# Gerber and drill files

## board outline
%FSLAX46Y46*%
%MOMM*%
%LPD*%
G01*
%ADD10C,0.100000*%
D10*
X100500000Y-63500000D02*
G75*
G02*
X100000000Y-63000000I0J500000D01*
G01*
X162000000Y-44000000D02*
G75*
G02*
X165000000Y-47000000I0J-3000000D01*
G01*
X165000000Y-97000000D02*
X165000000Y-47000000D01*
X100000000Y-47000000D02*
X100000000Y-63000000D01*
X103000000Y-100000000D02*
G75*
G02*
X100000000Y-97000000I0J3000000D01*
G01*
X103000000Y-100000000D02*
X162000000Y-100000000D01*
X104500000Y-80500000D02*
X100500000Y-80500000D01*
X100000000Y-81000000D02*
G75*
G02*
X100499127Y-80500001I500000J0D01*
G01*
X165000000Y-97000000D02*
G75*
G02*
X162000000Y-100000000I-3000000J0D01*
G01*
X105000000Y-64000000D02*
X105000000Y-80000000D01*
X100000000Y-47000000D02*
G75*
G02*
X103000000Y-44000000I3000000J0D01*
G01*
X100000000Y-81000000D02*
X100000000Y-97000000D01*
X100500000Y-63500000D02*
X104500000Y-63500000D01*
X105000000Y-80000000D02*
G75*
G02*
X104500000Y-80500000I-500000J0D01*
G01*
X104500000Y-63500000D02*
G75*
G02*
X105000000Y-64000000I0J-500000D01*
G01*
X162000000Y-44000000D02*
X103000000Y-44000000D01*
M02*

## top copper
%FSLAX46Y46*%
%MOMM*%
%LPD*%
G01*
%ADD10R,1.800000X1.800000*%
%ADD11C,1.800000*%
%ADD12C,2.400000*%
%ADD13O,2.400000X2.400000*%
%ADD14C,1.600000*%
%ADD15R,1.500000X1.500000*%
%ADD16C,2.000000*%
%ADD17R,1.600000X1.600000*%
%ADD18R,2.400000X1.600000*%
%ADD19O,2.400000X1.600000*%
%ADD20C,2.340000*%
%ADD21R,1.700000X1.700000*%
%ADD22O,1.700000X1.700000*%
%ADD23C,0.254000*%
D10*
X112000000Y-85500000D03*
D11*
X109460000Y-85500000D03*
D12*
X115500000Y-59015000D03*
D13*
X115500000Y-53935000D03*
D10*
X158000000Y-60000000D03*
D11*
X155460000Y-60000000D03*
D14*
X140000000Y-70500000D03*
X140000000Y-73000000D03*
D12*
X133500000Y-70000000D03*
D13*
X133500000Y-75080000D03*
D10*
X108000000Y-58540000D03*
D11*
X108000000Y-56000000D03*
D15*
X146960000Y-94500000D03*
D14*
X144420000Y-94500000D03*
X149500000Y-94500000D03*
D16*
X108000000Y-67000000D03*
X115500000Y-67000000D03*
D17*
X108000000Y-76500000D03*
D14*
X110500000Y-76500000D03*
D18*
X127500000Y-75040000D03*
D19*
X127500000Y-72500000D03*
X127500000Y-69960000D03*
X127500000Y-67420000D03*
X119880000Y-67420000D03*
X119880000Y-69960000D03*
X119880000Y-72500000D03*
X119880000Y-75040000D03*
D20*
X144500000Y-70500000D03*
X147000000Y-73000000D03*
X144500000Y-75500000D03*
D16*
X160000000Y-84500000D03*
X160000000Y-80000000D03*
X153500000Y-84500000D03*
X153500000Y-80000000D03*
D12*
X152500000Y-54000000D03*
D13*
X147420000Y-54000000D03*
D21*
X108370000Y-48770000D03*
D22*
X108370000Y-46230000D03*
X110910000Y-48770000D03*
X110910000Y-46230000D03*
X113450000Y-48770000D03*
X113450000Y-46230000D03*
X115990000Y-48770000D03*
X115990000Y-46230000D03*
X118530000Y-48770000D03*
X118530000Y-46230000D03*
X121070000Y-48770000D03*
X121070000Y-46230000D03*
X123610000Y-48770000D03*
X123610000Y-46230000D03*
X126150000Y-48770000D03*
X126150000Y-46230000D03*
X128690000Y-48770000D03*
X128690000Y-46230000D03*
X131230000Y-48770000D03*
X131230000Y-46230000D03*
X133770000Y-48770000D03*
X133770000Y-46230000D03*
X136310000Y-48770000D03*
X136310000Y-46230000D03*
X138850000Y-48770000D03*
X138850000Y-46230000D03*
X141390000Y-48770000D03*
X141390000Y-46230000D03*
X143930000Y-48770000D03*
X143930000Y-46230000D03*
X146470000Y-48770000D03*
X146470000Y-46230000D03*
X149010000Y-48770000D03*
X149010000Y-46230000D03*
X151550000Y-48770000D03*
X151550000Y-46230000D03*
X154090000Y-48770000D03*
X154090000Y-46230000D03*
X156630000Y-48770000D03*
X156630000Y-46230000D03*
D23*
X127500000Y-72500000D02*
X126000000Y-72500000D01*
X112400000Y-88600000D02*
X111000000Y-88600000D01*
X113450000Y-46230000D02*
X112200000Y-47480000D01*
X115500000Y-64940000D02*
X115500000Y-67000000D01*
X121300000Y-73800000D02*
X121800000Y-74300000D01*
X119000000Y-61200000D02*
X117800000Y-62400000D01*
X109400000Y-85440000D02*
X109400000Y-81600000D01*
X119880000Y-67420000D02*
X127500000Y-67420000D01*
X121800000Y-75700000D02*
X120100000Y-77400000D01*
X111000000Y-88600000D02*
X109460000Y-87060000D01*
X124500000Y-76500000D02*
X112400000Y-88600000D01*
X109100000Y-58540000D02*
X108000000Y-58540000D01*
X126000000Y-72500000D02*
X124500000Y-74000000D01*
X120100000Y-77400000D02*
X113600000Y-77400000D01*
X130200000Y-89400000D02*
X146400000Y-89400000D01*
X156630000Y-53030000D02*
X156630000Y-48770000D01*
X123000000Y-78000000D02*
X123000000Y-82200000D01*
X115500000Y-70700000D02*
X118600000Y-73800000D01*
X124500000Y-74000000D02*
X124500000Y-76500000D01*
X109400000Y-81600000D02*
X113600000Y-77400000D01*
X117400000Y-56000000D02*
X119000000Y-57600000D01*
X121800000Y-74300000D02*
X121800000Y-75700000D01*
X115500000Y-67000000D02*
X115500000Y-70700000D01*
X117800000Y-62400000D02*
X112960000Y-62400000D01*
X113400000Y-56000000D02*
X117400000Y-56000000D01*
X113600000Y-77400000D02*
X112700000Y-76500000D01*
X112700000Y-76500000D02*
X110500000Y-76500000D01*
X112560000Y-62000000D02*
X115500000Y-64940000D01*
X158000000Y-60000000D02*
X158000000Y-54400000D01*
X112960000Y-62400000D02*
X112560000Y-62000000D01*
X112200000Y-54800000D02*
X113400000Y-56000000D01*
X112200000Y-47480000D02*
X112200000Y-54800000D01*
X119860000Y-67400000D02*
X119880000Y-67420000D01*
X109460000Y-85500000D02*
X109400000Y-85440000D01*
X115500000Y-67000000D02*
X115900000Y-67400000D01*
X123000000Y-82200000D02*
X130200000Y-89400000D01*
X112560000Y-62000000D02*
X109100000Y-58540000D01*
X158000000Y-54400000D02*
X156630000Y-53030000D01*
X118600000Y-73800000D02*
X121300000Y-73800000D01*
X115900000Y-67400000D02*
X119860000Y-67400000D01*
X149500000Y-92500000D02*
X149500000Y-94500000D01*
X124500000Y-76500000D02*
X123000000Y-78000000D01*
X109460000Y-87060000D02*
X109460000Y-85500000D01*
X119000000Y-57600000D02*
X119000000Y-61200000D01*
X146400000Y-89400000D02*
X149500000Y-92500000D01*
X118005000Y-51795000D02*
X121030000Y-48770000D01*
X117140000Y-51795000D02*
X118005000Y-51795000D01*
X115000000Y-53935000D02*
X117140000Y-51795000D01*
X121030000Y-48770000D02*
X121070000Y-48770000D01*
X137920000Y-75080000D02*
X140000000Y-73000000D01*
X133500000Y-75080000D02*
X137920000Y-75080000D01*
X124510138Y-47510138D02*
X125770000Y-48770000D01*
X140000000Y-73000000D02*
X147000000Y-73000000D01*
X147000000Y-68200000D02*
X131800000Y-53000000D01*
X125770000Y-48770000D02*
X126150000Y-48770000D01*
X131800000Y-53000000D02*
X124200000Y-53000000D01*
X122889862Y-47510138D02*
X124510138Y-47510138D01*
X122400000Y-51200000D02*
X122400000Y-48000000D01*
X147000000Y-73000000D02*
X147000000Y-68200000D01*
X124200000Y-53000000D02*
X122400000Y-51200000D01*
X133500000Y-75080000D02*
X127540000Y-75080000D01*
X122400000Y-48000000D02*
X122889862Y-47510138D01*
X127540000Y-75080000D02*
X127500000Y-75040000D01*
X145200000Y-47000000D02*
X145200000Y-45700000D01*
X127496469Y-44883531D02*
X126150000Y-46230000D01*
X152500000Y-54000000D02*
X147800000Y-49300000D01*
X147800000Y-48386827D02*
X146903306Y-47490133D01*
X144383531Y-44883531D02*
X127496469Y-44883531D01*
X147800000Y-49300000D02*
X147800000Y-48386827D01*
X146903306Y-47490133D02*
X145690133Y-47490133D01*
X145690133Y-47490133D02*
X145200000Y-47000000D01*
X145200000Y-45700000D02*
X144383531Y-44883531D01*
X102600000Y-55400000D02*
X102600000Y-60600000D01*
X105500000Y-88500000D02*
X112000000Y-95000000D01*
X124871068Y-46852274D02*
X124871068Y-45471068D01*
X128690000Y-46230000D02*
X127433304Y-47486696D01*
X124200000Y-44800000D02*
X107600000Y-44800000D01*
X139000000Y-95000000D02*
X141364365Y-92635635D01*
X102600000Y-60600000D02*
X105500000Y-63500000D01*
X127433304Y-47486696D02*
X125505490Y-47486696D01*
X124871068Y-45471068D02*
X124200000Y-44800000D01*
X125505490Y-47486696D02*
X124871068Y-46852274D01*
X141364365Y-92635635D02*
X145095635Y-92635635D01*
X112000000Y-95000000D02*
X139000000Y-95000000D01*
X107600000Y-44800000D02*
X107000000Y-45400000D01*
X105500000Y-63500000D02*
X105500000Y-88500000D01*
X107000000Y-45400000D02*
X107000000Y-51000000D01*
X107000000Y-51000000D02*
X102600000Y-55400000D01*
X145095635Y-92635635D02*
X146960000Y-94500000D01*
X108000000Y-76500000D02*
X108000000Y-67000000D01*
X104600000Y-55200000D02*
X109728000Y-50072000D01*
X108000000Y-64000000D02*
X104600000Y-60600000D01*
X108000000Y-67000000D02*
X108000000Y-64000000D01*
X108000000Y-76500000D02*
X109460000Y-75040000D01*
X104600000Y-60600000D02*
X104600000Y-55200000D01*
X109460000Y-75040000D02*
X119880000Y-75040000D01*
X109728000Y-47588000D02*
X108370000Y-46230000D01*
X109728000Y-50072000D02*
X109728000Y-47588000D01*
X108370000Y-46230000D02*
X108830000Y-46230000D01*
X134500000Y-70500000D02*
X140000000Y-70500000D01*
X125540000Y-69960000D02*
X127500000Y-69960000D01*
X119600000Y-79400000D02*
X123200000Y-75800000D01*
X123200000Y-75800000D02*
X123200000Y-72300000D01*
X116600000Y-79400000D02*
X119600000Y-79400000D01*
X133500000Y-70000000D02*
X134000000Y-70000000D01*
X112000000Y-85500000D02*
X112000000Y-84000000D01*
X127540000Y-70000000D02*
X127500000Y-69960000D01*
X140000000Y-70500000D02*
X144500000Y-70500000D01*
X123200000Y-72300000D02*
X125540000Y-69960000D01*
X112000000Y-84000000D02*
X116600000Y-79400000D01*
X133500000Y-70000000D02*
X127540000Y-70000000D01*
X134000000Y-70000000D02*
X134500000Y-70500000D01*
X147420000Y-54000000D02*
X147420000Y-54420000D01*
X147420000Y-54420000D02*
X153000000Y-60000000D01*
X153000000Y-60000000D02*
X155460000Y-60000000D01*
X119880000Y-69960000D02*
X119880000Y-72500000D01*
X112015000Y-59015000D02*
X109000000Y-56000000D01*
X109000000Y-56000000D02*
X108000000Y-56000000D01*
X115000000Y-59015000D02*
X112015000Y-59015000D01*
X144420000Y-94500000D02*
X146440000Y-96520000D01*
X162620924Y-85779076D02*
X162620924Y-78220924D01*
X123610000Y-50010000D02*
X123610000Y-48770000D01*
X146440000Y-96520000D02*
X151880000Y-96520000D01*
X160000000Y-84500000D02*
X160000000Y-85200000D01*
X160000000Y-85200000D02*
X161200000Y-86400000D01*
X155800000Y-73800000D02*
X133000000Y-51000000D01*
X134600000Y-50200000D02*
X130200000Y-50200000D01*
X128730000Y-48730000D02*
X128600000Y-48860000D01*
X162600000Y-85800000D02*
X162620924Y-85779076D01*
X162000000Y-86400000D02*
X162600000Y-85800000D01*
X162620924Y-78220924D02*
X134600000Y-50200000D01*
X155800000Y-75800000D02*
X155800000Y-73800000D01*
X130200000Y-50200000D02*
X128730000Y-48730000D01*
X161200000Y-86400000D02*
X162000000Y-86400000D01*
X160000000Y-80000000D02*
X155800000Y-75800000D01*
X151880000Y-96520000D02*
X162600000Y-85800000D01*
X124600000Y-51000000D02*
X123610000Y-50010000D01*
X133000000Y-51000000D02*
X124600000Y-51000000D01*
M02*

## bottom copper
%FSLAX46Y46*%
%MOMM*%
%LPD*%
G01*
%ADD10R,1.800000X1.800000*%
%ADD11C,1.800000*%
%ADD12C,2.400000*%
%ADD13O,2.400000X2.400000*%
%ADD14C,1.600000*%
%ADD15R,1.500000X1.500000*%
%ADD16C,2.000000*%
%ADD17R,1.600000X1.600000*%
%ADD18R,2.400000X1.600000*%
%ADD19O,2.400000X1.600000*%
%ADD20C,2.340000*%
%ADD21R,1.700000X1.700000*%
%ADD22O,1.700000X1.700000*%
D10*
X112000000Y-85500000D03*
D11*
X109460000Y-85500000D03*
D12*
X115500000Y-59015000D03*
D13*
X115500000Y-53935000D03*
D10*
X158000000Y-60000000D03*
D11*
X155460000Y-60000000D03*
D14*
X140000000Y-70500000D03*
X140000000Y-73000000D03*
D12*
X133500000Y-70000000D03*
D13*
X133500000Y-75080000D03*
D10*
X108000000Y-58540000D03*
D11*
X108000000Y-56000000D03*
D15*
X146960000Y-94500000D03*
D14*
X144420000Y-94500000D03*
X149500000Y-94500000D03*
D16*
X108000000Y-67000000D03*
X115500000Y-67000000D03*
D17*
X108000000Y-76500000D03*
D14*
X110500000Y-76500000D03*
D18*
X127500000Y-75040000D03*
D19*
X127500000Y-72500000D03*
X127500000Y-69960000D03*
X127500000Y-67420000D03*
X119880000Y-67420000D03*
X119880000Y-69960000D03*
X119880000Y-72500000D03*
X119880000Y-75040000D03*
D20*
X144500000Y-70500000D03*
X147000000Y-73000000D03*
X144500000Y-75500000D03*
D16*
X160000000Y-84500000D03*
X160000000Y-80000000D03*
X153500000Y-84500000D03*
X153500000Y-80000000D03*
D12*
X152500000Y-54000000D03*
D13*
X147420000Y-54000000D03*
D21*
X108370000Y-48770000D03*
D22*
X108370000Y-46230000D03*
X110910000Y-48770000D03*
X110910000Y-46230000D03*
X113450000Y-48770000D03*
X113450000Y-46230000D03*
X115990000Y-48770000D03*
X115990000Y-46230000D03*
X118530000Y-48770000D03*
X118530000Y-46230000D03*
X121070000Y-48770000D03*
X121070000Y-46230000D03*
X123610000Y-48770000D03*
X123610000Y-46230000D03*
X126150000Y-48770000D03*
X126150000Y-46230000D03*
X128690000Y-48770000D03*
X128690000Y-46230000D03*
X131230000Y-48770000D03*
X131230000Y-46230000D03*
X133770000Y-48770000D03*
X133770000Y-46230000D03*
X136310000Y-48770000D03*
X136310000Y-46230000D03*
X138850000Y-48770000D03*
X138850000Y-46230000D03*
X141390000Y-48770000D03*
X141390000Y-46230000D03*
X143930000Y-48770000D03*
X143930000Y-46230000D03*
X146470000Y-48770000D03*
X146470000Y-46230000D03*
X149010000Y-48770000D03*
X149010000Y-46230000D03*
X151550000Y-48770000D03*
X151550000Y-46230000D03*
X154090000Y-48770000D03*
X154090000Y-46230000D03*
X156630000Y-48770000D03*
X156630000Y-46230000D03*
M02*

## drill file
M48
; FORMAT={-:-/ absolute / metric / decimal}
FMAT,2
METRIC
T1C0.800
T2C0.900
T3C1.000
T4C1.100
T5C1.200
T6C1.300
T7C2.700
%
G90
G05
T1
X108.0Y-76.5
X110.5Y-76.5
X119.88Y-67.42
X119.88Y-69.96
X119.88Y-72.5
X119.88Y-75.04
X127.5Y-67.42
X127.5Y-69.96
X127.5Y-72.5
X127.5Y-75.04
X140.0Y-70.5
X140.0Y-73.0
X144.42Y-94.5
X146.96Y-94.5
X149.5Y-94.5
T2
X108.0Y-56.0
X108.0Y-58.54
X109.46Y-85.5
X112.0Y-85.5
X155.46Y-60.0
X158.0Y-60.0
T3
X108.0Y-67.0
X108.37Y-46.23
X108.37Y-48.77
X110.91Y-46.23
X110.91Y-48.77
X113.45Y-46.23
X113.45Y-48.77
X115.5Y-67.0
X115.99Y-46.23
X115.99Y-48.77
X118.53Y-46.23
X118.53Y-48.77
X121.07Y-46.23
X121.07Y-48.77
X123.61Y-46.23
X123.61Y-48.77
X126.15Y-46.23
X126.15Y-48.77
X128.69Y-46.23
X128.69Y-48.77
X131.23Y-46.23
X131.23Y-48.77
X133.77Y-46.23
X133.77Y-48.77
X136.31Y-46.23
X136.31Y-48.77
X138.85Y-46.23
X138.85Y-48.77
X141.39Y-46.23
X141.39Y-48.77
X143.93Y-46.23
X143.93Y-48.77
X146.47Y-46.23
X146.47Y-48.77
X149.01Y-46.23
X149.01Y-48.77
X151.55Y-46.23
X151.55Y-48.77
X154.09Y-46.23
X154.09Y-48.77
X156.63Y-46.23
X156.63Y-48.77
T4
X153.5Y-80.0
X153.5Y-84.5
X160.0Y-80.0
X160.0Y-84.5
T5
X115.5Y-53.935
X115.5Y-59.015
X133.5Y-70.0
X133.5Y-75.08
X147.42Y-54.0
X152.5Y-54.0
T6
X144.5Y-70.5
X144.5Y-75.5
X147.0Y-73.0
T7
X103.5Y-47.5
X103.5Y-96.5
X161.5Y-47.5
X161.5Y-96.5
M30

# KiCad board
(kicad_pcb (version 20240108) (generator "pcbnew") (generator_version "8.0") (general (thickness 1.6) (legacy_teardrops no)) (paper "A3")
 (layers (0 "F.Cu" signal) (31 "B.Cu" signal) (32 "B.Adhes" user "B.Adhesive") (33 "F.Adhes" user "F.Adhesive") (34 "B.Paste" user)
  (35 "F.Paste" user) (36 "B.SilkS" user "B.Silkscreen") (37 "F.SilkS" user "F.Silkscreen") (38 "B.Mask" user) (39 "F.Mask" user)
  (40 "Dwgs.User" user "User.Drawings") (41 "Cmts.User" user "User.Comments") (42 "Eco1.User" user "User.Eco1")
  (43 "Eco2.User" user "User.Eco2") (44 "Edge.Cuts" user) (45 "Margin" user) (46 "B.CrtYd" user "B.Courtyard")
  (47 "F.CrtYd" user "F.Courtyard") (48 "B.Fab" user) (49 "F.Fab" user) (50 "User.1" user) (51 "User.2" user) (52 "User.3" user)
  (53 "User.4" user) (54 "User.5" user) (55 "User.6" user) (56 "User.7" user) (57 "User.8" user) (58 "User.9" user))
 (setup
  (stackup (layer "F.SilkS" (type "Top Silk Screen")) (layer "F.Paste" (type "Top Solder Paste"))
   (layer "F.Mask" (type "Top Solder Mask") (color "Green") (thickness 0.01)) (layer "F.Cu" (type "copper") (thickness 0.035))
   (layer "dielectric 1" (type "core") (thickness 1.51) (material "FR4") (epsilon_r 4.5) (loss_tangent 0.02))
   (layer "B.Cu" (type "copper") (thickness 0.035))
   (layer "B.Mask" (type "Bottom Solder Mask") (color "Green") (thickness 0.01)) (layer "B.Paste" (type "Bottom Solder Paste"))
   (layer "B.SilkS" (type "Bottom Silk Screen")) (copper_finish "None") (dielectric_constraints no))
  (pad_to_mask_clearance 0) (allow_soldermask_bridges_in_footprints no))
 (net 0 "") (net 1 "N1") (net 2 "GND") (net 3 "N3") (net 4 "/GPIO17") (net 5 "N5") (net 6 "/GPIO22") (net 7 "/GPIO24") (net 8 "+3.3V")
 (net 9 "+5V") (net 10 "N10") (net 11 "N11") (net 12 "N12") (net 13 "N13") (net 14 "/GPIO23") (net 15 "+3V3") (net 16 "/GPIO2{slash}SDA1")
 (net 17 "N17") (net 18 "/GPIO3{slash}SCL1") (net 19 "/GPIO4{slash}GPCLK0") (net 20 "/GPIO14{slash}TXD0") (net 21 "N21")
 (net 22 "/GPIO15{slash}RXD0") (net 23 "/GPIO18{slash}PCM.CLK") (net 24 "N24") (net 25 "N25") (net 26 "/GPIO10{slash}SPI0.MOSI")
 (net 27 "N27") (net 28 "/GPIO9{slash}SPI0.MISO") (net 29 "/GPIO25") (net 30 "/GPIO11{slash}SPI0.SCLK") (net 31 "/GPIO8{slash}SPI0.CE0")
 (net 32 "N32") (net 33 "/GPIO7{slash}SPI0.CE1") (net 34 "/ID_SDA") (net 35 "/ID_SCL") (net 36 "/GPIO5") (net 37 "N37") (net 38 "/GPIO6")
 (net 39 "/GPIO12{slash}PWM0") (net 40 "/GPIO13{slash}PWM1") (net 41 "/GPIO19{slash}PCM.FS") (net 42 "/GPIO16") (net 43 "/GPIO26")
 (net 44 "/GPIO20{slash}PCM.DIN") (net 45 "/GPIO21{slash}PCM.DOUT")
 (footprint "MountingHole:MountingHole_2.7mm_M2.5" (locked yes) (layer "F.Cu") (at 161.5 47.5)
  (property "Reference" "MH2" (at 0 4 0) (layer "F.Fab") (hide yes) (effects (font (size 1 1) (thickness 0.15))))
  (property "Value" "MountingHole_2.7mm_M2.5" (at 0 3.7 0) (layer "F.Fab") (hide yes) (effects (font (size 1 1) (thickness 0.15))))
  (pad "" np_thru_hole circle (at 0 0) (size 2.7 2.7) (drill 2.7) (layers "*.Cu" "*.Mask")))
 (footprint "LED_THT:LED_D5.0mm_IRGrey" (layer "F.Cu") (at 112 85.5 180)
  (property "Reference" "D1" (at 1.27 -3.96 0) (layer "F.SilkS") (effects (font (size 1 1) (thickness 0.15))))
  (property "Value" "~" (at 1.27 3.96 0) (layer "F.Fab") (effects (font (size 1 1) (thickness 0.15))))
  (pad "1" thru_hole rect (at 0 0 180) (size 1.8 1.8) (drill 0.9) (layers "*.Cu" "*.Mask") (remove_unused_layers no) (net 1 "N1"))
  (pad "2" thru_hole circle (at 2.54 0 180) (size 1.8 1.8) (drill 0.9) (layers "*.Cu" "*.Mask") (remove_unused_layers no) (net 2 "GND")))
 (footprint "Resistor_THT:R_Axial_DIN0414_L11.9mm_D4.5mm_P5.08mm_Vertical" (layer "F.Cu") (at 115.5 59.015 90)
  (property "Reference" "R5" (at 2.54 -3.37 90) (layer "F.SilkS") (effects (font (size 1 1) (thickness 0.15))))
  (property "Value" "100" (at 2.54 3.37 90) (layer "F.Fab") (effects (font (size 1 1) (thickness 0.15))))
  (pad "1" thru_hole circle (at 0 0 90) (size 2.4 2.4) (drill 1.2) (layers "*.Cu" "*.Mask") (remove_unused_layers no) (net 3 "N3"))
  (pad "2" thru_hole oval (at 5.08 0 90) (size 2.4 2.4) (drill 1.2) (layers "*.Cu" "*.Mask") (remove_unused_layers no) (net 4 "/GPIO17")))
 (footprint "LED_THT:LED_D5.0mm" (layer "F.Cu") (at 158 60 180)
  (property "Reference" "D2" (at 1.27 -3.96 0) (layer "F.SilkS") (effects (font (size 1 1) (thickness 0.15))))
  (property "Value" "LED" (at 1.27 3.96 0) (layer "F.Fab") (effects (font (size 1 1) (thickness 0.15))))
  (pad "1" thru_hole rect (at 0 0 180) (size 1.8 1.8) (drill 0.9) (layers "*.Cu" "*.Mask") (remove_unused_layers no) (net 2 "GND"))
  (pad "2" thru_hole circle (at 2.54 0 180) (size 1.8 1.8) (drill 0.9) (layers "*.Cu" "*.Mask") (remove_unused_layers no) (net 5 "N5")))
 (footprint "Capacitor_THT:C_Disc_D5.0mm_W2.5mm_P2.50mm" (layer "F.Cu") (at 140 70.5 -90)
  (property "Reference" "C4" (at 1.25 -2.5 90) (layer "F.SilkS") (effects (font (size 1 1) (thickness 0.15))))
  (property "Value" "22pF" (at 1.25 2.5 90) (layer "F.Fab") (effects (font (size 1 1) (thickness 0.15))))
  (pad "1" thru_hole circle (at 0 0 270) (size 1.6 1.6) (drill 0.8) (layers "*.Cu" "*.Mask") (remove_unused_layers no) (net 1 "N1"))
  (pad "2" thru_hole circle (at 2.5 0 270) (size 1.6 1.6) (drill 0.8) (layers "*.Cu" "*.Mask") (remove_unused_layers no) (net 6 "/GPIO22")))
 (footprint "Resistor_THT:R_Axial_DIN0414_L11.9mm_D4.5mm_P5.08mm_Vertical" (layer "F.Cu") (at 133.5 70 -90)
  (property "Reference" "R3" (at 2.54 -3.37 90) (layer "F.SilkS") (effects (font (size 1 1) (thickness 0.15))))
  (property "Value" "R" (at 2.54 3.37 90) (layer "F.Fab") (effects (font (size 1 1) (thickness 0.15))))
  (pad "1" thru_hole circle (at 0 0 270) (size 2.4 2.4) (drill 1.2) (layers "*.Cu" "*.Mask") (remove_unused_layers no) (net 1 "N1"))
  (pad "2" thru_hole oval (at 5.08 0 270) (size 2.4 2.4) (drill 1.2) (layers "*.Cu" "*.Mask") (remove_unused_layers no) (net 6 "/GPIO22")))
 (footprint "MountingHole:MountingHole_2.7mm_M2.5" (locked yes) (layer "F.Cu") (at 103.5 96.5)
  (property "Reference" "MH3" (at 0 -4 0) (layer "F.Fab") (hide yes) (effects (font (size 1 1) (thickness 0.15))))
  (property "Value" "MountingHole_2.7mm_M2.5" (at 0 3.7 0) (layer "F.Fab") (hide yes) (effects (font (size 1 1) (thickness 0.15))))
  (pad "" np_thru_hole circle (at 0 0) (size 2.7 2.7) (drill 2.7) (layers "*.Cu" "*.Mask")))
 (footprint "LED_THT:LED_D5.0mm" (layer "F.Cu") (at 108 58.54 90)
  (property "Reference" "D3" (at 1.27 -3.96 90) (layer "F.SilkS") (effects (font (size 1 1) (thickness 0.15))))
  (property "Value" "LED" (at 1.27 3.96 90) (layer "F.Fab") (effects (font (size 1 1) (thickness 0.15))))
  (pad "1" thru_hole rect (at 0 0 90) (size 1.8 1.8) (drill 0.9) (layers "*.Cu" "*.Mask") (remove_unused_layers no) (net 2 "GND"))
  (pad "2" thru_hole circle (at 2.54 0 90) (size 1.8 1.8) (drill 0.9) (layers "*.Cu" "*.Mask") (remove_unused_layers no) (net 3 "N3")))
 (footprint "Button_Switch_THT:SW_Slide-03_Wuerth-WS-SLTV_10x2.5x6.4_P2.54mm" (layer "F.Cu") (at 146.96 94.5)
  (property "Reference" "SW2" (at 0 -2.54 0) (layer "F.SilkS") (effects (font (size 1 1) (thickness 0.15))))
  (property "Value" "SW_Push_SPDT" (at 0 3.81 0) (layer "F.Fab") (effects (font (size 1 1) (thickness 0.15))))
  (pad "1" thru_hole rect (at 0 0) (size 1.5 1.5) (drill 0.8) (layers "*.Cu" "*.Mask") (remove_unused_layers no) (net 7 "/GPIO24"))
  (pad "2" thru_hole circle (at -2.54 0) (size 1.6 1.6) (drill 0.8) (layers "*.Cu" "*.Mask") (remove_unused_layers no) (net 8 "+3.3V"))
  (pad "3" thru_hole circle (at 2.54 0) (size 1.6 1.6) (drill 0.8) (layers "*.Cu" "*.Mask") (remove_unused_layers no) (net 2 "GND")))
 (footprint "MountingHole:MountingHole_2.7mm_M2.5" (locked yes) (layer "F.Cu") (at 103.5 47.5)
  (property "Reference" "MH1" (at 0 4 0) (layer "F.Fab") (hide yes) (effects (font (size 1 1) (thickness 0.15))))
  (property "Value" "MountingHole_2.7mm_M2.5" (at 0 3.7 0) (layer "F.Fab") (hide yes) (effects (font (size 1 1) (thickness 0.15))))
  (pad "" np_thru_hole circle (at 0 0) (size 2.7 2.7) (drill 2.7) (layers "*.Cu" "*.Mask")))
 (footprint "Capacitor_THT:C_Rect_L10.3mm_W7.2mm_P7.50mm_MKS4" (layer "F.Cu") (at 108 67)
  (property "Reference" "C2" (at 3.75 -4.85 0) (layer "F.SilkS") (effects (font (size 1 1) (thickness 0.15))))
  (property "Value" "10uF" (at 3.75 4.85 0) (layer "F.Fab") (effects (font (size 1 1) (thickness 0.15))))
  (pad "1" thru_hole circle (at 0 0) (size 2 2) (drill 1) (layers "*.Cu" "*.Mask") (remove_unused_layers no) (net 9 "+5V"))
  (pad "2" thru_hole circle (at 7.5 0) (size 2 2) (drill 1) (layers "*.Cu" "*.Mask") (remove_unused_layers no) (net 2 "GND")))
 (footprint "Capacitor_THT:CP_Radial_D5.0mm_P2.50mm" (layer "F.Cu") (at 108 76.5)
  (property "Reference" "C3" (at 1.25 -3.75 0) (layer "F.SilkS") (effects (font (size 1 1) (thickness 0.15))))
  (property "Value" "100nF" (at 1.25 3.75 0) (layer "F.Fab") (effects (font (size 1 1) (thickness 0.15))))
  (pad "1" thru_hole rect (at 0 0) (size 1.6 1.6) (drill 0.8) (layers "*.Cu" "*.Mask") (remove_unused_layers no) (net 9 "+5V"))
  (pad "2" thru_hole circle (at 2.5 0) (size 1.6 1.6) (drill 0.8) (layers "*.Cu" "*.Mask") (remove_unused_layers no) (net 2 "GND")))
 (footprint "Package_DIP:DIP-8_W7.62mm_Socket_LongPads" (layer "F.Cu") (at 127.5 75.04 180)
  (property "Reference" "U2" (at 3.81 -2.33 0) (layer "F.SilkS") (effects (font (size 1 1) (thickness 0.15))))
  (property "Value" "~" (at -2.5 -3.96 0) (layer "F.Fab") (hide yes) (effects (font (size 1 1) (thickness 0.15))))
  (pad "1" thru_hole rect (at 0 0 180) (size 2.4 1.6) (drill 0.8) (layers "*.Cu" "*.Mask") (remove_unused_layers no) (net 6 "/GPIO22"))
  (pad "2" thru_hole oval (at 0 2.54 180) (size 2.4 1.6) (drill 0.8) (layers "*.Cu" "*.Mask") (remove_unused_layers no) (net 2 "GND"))
  (pad "3" thru_hole oval (at 0 5.08 180) (size 2.4 1.6) (drill 0.8) (layers "*.Cu" "*.Mask") (remove_unused_layers no) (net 1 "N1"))
  (pad "4" thru_hole oval (at 0 7.62 180) (size 2.4 1.6) (drill 0.8) (layers "*.Cu" "*.Mask") (remove_unused_layers no) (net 2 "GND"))
  (pad "5" thru_hole oval (at 7.62 7.62 180) (size 2.4 1.6) (drill 0.8) (layers "*.Cu" "*.Mask") (remove_unused_layers no) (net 2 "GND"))
  (pad "6" thru_hole oval (at 7.62 5.08 180) (size 2.4 1.6) (drill 0.8) (layers "*.Cu" "*.Mask") (remove_unused_layers no) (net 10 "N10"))
  (pad "7" thru_hole oval (at 7.62 2.54 180) (size 2.4 1.6) (drill 0.8) (layers "*.Cu" "*.Mask") (remove_unused_layers no) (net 10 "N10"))
  (pad "8" thru_hole oval (at 7.62 0 180) (size 2.4 1.6) (drill 0.8) (layers "*.Cu" "*.Mask") (remove_unused_layers no) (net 9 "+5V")))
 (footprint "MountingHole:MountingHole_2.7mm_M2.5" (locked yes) (layer "F.Cu") (at 161.5 96.5)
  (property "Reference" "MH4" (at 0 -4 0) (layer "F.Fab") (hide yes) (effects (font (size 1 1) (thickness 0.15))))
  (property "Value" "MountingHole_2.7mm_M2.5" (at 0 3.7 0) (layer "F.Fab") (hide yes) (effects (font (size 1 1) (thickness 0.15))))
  (pad "" np_thru_hole circle (at 0 0) (size 2.7 2.7) (drill 2.7) (layers "*.Cu" "*.Mask")))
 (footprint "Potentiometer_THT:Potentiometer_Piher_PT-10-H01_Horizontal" (layer "F.Cu") (at 144.5 70.5)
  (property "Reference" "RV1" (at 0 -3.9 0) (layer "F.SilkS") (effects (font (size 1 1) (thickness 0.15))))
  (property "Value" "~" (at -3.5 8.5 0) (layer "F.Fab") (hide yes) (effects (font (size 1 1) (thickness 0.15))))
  (pad "1" thru_hole circle (at 0 0) (size 2.34 2.34) (drill 1.3) (layers "*.Cu" "*.Mask") (remove_unused_layers no) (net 1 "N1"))
  (pad "2" thru_hole circle (at 2.5 2.5) (size 2.34 2.34) (drill 1.3) (layers "*.Cu" "*.Mask") (remove_unused_layers no) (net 6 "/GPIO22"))
  (pad "3" thru_hole circle (at 0 5) (size 2.34 2.34) (drill 1.3) (layers "*.Cu" "*.Mask") (remove_unused_layers no) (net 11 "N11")))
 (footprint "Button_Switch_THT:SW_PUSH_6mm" (layer "F.Cu") (at 160 84.5 180)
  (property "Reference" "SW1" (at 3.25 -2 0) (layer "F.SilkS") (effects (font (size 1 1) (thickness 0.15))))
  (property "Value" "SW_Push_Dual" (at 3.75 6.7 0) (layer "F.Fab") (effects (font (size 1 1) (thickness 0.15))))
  (pad "1" thru_hole circle (at 0 0 270) (size 2 2) (drill 1.1) (layers "*.Cu" "*.Mask") (remove_unused_layers no) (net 8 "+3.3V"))
  (pad "2" thru_hole circle (at 0 4.5 270) (size 2 2) (drill 1.1) (layers "*.Cu" "*.Mask") (remove_unused_layers no) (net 8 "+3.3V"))
  (pad "3" thru_hole circle (at 6.5 0 270) (size 2 2) (drill 1.1) (layers "*.Cu" "*.Mask") (remove_unused_layers no) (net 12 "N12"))
  (pad "4" thru_hole circle (at 6.5 4.5 270) (size 2 2) (drill 1.1) (layers "*.Cu" "*.Mask") (remove_unused_layers no) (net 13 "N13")))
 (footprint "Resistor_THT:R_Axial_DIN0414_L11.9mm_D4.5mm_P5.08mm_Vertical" (layer "F.Cu") (at 152.5 54 180)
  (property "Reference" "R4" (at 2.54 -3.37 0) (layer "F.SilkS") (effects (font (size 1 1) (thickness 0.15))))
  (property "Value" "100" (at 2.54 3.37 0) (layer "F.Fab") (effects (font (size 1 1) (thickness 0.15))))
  (pad "1" thru_hole circle (at 0 0 180) (size 2.4 2.4) (drill 1.2) (layers "*.Cu" "*.Mask") (remove_unused_layers no) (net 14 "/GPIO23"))
  (pad "2" thru_hole oval (at 5.08 0 180) (size 2.4 2.4) (drill 1.2) (layers "*.Cu" "*.Mask") (remove_unused_layers no) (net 5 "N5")))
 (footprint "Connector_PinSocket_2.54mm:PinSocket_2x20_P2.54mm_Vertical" (layer "B.Cu") (at 108.37 48.77 -90)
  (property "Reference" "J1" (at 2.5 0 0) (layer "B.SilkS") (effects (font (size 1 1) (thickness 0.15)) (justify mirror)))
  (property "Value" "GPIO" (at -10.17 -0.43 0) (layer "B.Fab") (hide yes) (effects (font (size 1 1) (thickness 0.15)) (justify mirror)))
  (pad "1" thru_hole rect (at 0 0 270) (size 1.7 1.7) (drill 1) (layers "*.Cu" "*.Mask") (remove_unused_layers no) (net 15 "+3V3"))
  (pad "2" thru_hole oval (at -2.54 0 270) (size 1.7 1.7) (drill 1) (layers "*.Cu" "*.Mask") (remove_unused_layers no) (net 9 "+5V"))
  (pad "3" thru_hole oval (at 0 -2.54 270) (size 1.7 1.7) (drill 1) (layers "*.Cu" "*.Mask") (remove_unused_layers no)
   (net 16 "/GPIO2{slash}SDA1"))
  (pad "4" thru_hole oval (at -2.54 -2.54 270) (size 1.7 1.7) (drill 1) (layers "*.Cu" "*.Mask") (remove_unused_layers no) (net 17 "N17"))
  (pad "5" thru_hole oval (at 0 -5.08 270) (size 1.7 1.7) (drill 1) (layers "*.Cu" "*.Mask") (remove_unused_layers no)
   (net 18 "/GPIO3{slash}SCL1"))
  (pad "6" thru_hole oval (at -2.54 -5.08 270) (size 1.7 1.7) (drill 1) (layers "*.Cu" "*.Mask") (remove_unused_layers no) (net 2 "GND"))
  (pad "7" thru_hole oval (at 0 -7.62 270) (size 1.7 1.7) (drill 1) (layers "*.Cu" "*.Mask") (remove_unused_layers no)
   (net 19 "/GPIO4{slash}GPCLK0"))
  (pad "8" thru_hole oval (at -2.54 -7.62 270) (size 1.7 1.7) (drill 1) (layers "*.Cu" "*.Mask") (remove_unused_layers no)
   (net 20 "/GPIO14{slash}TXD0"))
  (pad "9" thru_hole oval (at 0 -10.16 270) (size 1.7 1.7) (drill 1) (layers "*.Cu" "*.Mask") (remove_unused_layers no) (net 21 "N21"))
  (pad "10" thru_hole oval (at -2.54 -10.16 270) (size 1.7 1.7) (drill 1) (layers "*.Cu" "*.Mask") (remove_unused_layers no)
   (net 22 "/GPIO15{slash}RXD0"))
  (pad "11" thru_hole oval (at 0 -12.7 270) (size 1.7 1.7) (drill 1) (layers "*.Cu" "*.Mask") (remove_unused_layers no) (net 4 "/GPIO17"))
  (pad "12" thru_hole oval (at -2.54 -12.7 270) (size 1.7 1.7) (drill 1) (layers "*.Cu" "*.Mask") (remove_unused_layers no)
   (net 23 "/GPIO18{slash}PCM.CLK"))
  (pad "13" thru_hole oval (at 0 -15.24 270) (size 1.7 1.7) (drill 1) (layers "*.Cu" "*.Mask") (remove_unused_layers no) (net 8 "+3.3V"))
  (pad "14" thru_hole oval (at -2.54 -15.24 270) (size 1.7 1.7) (drill 1) (layers "*.Cu" "*.Mask") (remove_unused_layers no) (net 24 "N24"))
  (pad "15" thru_hole oval (at 0 -17.78 270) (size 1.7 1.7) (drill 1) (layers "*.Cu" "*.Mask") (remove_unused_layers no) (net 6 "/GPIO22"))
  (pad "16" thru_hole oval (at -2.54 -17.78 270) (size 1.7 1.7) (drill 1) (layers "*.Cu" "*.Mask") (remove_unused_layers no)
   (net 14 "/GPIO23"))
  (pad "17" thru_hole oval (at 0 -20.32 270) (size 1.7 1.7) (drill 1) (layers "*.Cu" "*.Mask") (remove_unused_layers no) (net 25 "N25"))
  (pad "18" thru_hole oval (at -2.54 -20.32 270) (size 1.7 1.7) (drill 1) (layers "*.Cu" "*.Mask") (remove_unused_layers no)
   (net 7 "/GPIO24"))
  (pad "19" thru_hole oval (at 0 -22.86 270) (size 1.7 1.7) (drill 1) (layers "*.Cu" "*.Mask") (remove_unused_layers no)
   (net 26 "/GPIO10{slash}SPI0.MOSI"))
  (pad "20" thru_hole oval (at -2.54 -22.86 270) (size 1.7 1.7) (drill 1) (layers "*.Cu" "*.Mask") (remove_unused_layers no) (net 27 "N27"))
  (pad "21" thru_hole oval (at 0 -25.4 270) (size 1.7 1.7) (drill 1) (layers "*.Cu" "*.Mask") (remove_unused_layers no)
   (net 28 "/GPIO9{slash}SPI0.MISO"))
  (pad "22" thru_hole oval (at -2.54 -25.4 270) (size 1.7 1.7) (drill 1) (layers "*.Cu" "*.Mask") (remove_unused_layers no)
   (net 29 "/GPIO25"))
  (pad "23" thru_hole oval (at 0 -27.94 270) (size 1.7 1.7) (drill 1) (layers "*.Cu" "*.Mask") (remove_unused_layers no)
   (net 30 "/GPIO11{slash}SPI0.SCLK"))
  (pad "24" thru_hole oval (at -2.54 -27.94 270) (size 1.7 1.7) (drill 1) (layers "*.Cu" "*.Mask") (remove_unused_layers no)
   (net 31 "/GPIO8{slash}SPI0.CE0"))
  (pad "25" thru_hole oval (at 0 -30.48 270) (size 1.7 1.7) (drill 1) (layers "*.Cu" "*.Mask") (remove_unused_layers no) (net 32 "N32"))
  (pad "26" thru_hole oval (at -2.54 -30.48 270) (size 1.7 1.7) (drill 1) (layers "*.Cu" "*.Mask") (remove_unused_layers no)
   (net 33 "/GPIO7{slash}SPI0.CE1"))
  (pad "27" thru_hole oval (at 0 -33.02 270) (size 1.7 1.7) (drill 1) (layers "*.Cu" "*.Mask") (remove_unused_layers no) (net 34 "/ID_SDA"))
  (pad "28" thru_hole oval (at -2.54 -33.02 270) (size 1.7 1.7) (drill 1) (layers "*.Cu" "*.Mask") (remove_unused_layers no)
   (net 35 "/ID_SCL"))
  (pad "29" thru_hole oval (at 0 -35.56 270) (size 1.7 1.7) (drill 1) (layers "*.Cu" "*.Mask") (remove_unused_layers no) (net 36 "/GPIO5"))
  (pad "30" thru_hole oval (at -2.54 -35.56 270) (size 1.7 1.7) (drill 1) (layers "*.Cu" "*.Mask") (remove_unused_layers no) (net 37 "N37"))
  (pad "31" thru_hole oval (at 0 -38.1 270) (size 1.7 1.7) (drill 1) (layers "*.Cu" "*.Mask") (remove_unused_layers no) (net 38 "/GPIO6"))
  (pad "32" thru_hole oval (at -2.54 -38.1 270) (size 1.7 1.7) (drill 1) (layers "*.Cu" "*.Mask") (remove_unused_layers no)
   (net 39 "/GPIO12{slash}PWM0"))
  (pad "33" thru_hole oval (at 0 -40.64 270) (size 1.7 1.7) (drill 1) (layers "*.Cu" "*.Mask") (remove_unused_layers no)
   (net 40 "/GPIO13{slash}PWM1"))
  (pad "34" thru_hole oval (at -2.54 -40.64 270) (size 1.7 1.7) (drill 1) (layers "*.Cu" "*.Mask") (remove_unused_layers no) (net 2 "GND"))
  (pad "35" thru_hole oval (at 0 -43.18 270) (size 1.7 1.7) (drill 1) (layers "*.Cu" "*.Mask") (remove_unused_layers no)
   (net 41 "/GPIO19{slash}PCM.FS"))
  (pad "36" thru_hole oval (at -2.54 -43.18 270) (size 1.7 1.7) (drill 1) (layers "*.Cu" "*.Mask") (remove_unused_layers no)
   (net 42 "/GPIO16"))
  (pad "37" thru_hole oval (at 0 -45.72 270) (size 1.7 1.7) (drill 1) (layers "*.Cu" "*.Mask") (remove_unused_layers no) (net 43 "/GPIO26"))
  (pad "38" thru_hole oval (at -2.54 -45.72 270) (size 1.7 1.7) (drill 1) (layers "*.Cu" "*.Mask") (remove_unused_layers no)
   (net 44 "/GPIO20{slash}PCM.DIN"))
  (pad "39" thru_hole oval (at 0 -48.26 270) (size 1.7 1.7) (drill 1) (layers "*.Cu" "*.Mask") (remove_unused_layers no) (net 2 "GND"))
  (pad "40" thru_hole oval (at -2.54 -48.26 270) (size 1.7 1.7) (drill 1) (layers "*.Cu" "*.Mask") (remove_unused_layers no)
   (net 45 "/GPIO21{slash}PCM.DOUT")))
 (gr_arc (start 100.5 63.5) (mid 100.146447 63.353553) (end 100 63) (stroke (width 0.1) (type solid)) (layer "Edge.Cuts"))
 (gr_arc (start 162 44) (mid 164.12132 44.87868) (end 165 47) (stroke (width 0.1) (type solid)) (layer "Edge.Cuts"))
 (gr_line (start 165 97) (end 165 47) (stroke (width 0.1) (type solid)) (layer "Edge.Cuts"))
 (gr_line (start 100 47) (end 100 63) (stroke (width 0.1) (type solid)) (layer "Edge.Cuts"))
 (gr_arc (start 103 100) (mid 100.87868 99.12132) (end 100 97) (stroke (width 0.1) (type solid)) (layer "Edge.Cuts"))
 (gr_line (start 103 100) (end 162 100) (stroke (width 0.1) (type solid)) (layer "Edge.Cuts"))
 (gr_line (start 104.5 80.5) (end 100.5 80.5) (stroke (width 0.1) (type solid)) (layer "Edge.Cuts"))
 (gr_arc (start 100 81) (mid 100.146138 80.646755) (end 100.499127 80.500001) (stroke (width 0.1) (type solid)) (layer "Edge.Cuts"))
 (gr_arc (start 165 97) (mid 164.12132 99.12132) (end 162 100) (stroke (width 0.1) (type solid)) (layer "Edge.Cuts"))
 (gr_line (start 105 64) (end 105 80) (stroke (width 0.1) (type solid)) (layer "Edge.Cuts"))
 (gr_arc (start 100 47) (mid 100.87868 44.87868) (end 103 44) (stroke (width 0.1) (type solid)) (layer "Edge.Cuts"))
 (gr_line (start 100 81) (end 100 97) (stroke (width 0.1) (type solid)) (layer "Edge.Cuts"))
 (gr_line (start 100.5 63.5) (end 104.5 63.5) (stroke (width 0.1) (type solid)) (layer "Edge.Cuts"))
 (gr_arc (start 105 80) (mid 104.853553 80.353553) (end 104.5 80.5) (stroke (width 0.1) (type solid)) (layer "Edge.Cuts"))
 (gr_arc (start 104.5 63.5) (mid 104.853553 63.646447) (end 105 64) (stroke (width 0.1) (type solid)) (layer "Edge.Cuts"))
 (gr_line (start 162 44) (end 103 44) (stroke (width 0.1) (type solid)) (layer "Edge.Cuts"))
 (segment (start 127.5 72.5) (end 126 72.5) (width 0.254) (layer "F.Cu") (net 2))
 (segment (start 112.4 88.6) (end 111 88.6) (width 0.254) (layer "F.Cu") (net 2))
 (segment (start 113.45 46.23) (end 112.2 47.48) (width 0.254) (layer "F.Cu") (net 2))
 (segment (start 115.5 64.94) (end 115.5 67) (width 0.254) (layer "F.Cu") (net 2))
 (segment (start 121.3 73.8) (end 121.8 74.3) (width 0.254) (layer "F.Cu") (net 2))
 (segment (start 119 61.2) (end 117.8 62.4) (width 0.254) (layer "F.Cu") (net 2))
 (segment (start 109.4 85.44) (end 109.4 81.6) (width 0.254) (layer "F.Cu") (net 2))
 (segment (start 119.88 67.42) (end 127.5 67.42) (width 0.254) (layer "F.Cu") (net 2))
 (segment (start 121.8 75.7) (end 120.1 77.4) (width 0.254) (layer "F.Cu") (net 2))
 (segment (start 111 88.6) (end 109.46 87.06) (width 0.254) (layer "F.Cu") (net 2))
 (segment (start 124.5 76.5) (end 112.4 88.6) (width 0.254) (layer "F.Cu") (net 2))
 (segment (start 109.1 58.54) (end 108 58.54) (width 0.254) (layer "F.Cu") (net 2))
 (segment (start 126 72.5) (end 124.5 74) (width 0.254) (layer "F.Cu") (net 2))
 (segment (start 120.1 77.4) (end 113.6 77.4) (width 0.254) (layer "F.Cu") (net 2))
 (segment (start 130.2 89.4) (end 146.4 89.4) (width 0.254) (layer "F.Cu") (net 2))
 (segment (start 156.63 53.03) (end 156.63 48.77) (width 0.254) (layer "F.Cu") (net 2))
 (segment (start 123 78) (end 123 82.2) (width 0.254) (layer "F.Cu") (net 2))
 (segment (start 115.5 70.7) (end 118.6 73.8) (width 0.254) (layer "F.Cu") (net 2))
 (segment (start 124.5 74) (end 124.5 76.5) (width 0.254) (layer "F.Cu") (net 2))
 (segment (start 109.4 81.6) (end 113.6 77.4) (width 0.254) (layer "F.Cu") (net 2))
 (segment (start 117.4 56) (end 119 57.6) (width 0.254) (layer "F.Cu") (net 2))
 (segment (start 121.8 74.3) (end 121.8 75.7) (width 0.254) (layer "F.Cu") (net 2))
 (segment (start 115.5 67) (end 115.5 70.7) (width 0.254) (layer "F.Cu") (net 2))
 (segment (start 117.8 62.4) (end 112.96 62.4) (width 0.254) (layer "F.Cu") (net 2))
 (segment (start 113.4 56) (end 117.4 56) (width 0.254) (layer "F.Cu") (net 2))
 (segment (start 113.6 77.4) (end 112.7 76.5) (width 0.254) (layer "F.Cu") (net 2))
 (segment (start 112.7 76.5) (end 110.5 76.5) (width 0.254) (layer "F.Cu") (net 2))
 (segment (start 112.56 62) (end 115.5 64.94) (width 0.254) (layer "F.Cu") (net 2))
 (segment (start 158 60) (end 158 54.4) (width 0.254) (layer "F.Cu") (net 2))
 (segment (start 112.96 62.4) (end 112.56 62) (width 0.254) (layer "F.Cu") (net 2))
 (segment (start 112.2 54.8) (end 113.4 56) (width 0.254) (layer "F.Cu") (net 2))
 (segment (start 112.2 47.48) (end 112.2 54.8) (width 0.254) (layer "F.Cu") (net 2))
 (segment (start 119.86 67.4) (end 119.88 67.42) (width 0.254) (layer "F.Cu") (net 2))
 (segment (start 109.46 85.5) (end 109.4 85.44) (width 0.254) (layer "F.Cu") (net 2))
 (segment (start 115.5 67) (end 115.9 67.4) (width 0.254) (layer "F.Cu") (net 2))
 (segment (start 123 82.2) (end 130.2 89.4) (width 0.254) (layer "F.Cu") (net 2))
 (segment (start 112.56 62) (end 109.1 58.54) (width 0.254) (layer "F.Cu") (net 2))
 (segment (start 158 54.4) (end 156.63 53.03) (width 0.254) (layer "F.Cu") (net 2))
 (segment (start 118.6 73.8) (end 121.3 73.8) (width 0.254) (layer "F.Cu") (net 2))
 (segment (start 115.9 67.4) (end 119.86 67.4) (width 0.254) (layer "F.Cu") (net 2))
 (segment (start 149.5 92.5) (end 149.5 94.5) (width 0.254) (layer "F.Cu") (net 2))
 (segment (start 124.5 76.5) (end 123 78) (width 0.254) (layer "F.Cu") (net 2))
 (segment (start 109.46 87.06) (end 109.46 85.5) (width 0.254) (layer "F.Cu") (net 2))
 (segment (start 119 57.6) (end 119 61.2) (width 0.254) (layer "F.Cu") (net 2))
 (segment (start 146.4 89.4) (end 149.5 92.5) (width 0.254) (layer "F.Cu") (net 2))
 (segment (start 118.005 51.795) (end 121.03 48.77) (width 0.254) (layer "F.Cu") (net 4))
 (segment (start 117.14 51.795) (end 118.005 51.795) (width 0.254) (layer "F.Cu") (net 4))
 (segment (start 115 53.935) (end 117.14 51.795) (width 0.254) (layer "F.Cu") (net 4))
 (segment (start 121.03 48.77) (end 121.07 48.77) (width 0.254) (layer "F.Cu") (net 4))
 (segment (start 137.92 75.08) (end 140 73) (width 0.254) (layer "F.Cu") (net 6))
 (segment (start 133.5 75.08) (end 137.92 75.08) (width 0.254) (layer "F.Cu") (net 6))
 (segment (start 124.510138 47.510138) (end 125.77 48.77) (width 0.254) (layer "F.Cu") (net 6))
 (segment (start 140 73) (end 147 73) (width 0.254) (layer "F.Cu") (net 6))
 (segment (start 147 68.2) (end 131.8 53) (width 0.254) (layer "F.Cu") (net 6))
 (segment (start 125.77 48.77) (end 126.15 48.77) (width 0.254) (layer "F.Cu") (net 6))
 (segment (start 131.8 53) (end 124.2 53) (width 0.254) (layer "F.Cu") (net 6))
 (segment (start 122.889862 47.510138) (end 124.510138 47.510138) (width 0.254) (layer "F.Cu") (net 6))
 (segment (start 122.4 51.2) (end 122.4 48) (width 0.254) (layer "F.Cu") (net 6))
 (segment (start 147 73) (end 147 68.2) (width 0.254) (layer "F.Cu") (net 6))
 (segment (start 124.2 53) (end 122.4 51.2) (width 0.254) (layer "F.Cu") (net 6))
 (segment (start 133.5 75.08) (end 127.54 75.08) (width 0.254) (layer "F.Cu") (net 6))
 (segment (start 122.4 48) (end 122.889862 47.510138) (width 0.254) (layer "F.Cu") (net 6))
 (segment (start 127.54 75.08) (end 127.5 75.04) (width 0.254) (layer "F.Cu") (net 6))
 (segment (start 145.2 47) (end 145.2 45.7) (width 0.254) (layer "F.Cu") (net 14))
 (segment (start 127.496469 44.883531) (end 126.15 46.23) (width 0.254) (layer "F.Cu") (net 14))
 (segment (start 152.5 54) (end 147.8 49.3) (width 0.254) (layer "F.Cu") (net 14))
 (segment (start 147.8 48.386827) (end 146.903306 47.490133) (width 0.254) (layer "F.Cu") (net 14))
 (segment (start 144.383531 44.883531) (end 127.496469 44.883531) (width 0.254) (layer "F.Cu") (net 14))
 (segment (start 147.8 49.3) (end 147.8 48.386827) (width 0.254) (layer "F.Cu") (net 14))
 (segment (start 146.903306 47.490133) (end 145.690133 47.490133) (width 0.254) (layer "F.Cu") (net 14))
 (segment (start 145.690133 47.490133) (end 145.2 47) (width 0.254) (layer "F.Cu") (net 14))
 (segment (start 145.2 45.7) (end 144.383531 44.883531) (width 0.254) (layer "F.Cu") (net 14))
 (segment (start 102.6 55.4) (end 102.6 60.6) (width 0.254) (layer "F.Cu") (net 7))
 (segment (start 105.5 88.5) (end 112 95) (width 0.254) (layer "F.Cu") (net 7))
 (segment (start 124.871068 46.852274) (end 124.871068 45.471068) (width 0.254) (layer "F.Cu") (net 7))
 (segment (start 128.69 46.23) (end 127.433304 47.486696) (width 0.254) (layer "F.Cu") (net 7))
 (segment (start 124.2 44.8) (end 107.6 44.8) (width 0.254) (layer "F.Cu") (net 7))
 (segment (start 139 95) (end 141.364365 92.635635) (width 0.254) (layer "F.Cu") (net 7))
 (segment (start 102.6 60.6) (end 105.5 63.5) (width 0.254) (layer "F.Cu") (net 7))
 (segment (start 127.433304 47.486696) (end 125.50549 47.486696) (width 0.254) (layer "F.Cu") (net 7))
 (segment (start 124.871068 45.471068) (end 124.2 44.8) (width 0.254) (layer "F.Cu") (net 7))
 (segment (start 125.50549 47.486696) (end 124.871068 46.852274) (width 0.254) (layer "F.Cu") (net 7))
 (segment (start 141.364365 92.635635) (end 145.095635 92.635635) (width 0.254) (layer "F.Cu") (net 7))
 (segment (start 112 95) (end 139 95) (width 0.254) (layer "F.Cu") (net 7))
 (segment (start 107.6 44.8) (end 107 45.4) (width 0.254) (layer "F.Cu") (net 7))
 (segment (start 105.5 63.5) (end 105.5 88.5) (width 0.254) (layer "F.Cu") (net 7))
 (segment (start 107 45.4) (end 107 51) (width 0.254) (layer "F.Cu") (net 7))
 (segment (start 107 51) (end 102.6 55.4) (width 0.254) (layer "F.Cu") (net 7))
 (segment (start 145.095635 92.635635) (end 146.96 94.5) (width 0.254) (layer "F.Cu") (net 7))
 (segment (start 108 76.5) (end 108 67) (width 0.254) (layer "F.Cu") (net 9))
 (segment (start 104.6 55.2) (end 109.728 50.072) (width 0.254) (layer "F.Cu") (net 9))
 (segment (start 108 64) (end 104.6 60.6) (width 0.254) (layer "F.Cu") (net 9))
 (segment (start 108 67) (end 108 64) (width 0.254) (layer "F.Cu") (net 9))
 (segment (start 108 76.5) (end 109.46 75.04) (width 0.254) (layer "F.Cu") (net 9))
 (segment (start 104.6 60.6) (end 104.6 55.2) (width 0.254) (layer "F.Cu") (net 9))
 (segment (start 109.46 75.04) (end 119.88 75.04) (width 0.254) (layer "F.Cu") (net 9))
 (segment (start 109.728 47.588) (end 108.37 46.23) (width 0.254) (layer "F.Cu") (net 9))
 (segment (start 109.728 50.072) (end 109.728 47.588) (width 0.254) (layer "F.Cu") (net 9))
 (segment (start 108.37 46.23) (end 108.83 46.23) (width 0.254) (layer "F.Cu") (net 9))
 (segment (start 134.5 70.5) (end 140 70.5) (width 0.254) (layer "F.Cu") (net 1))
 (segment (start 125.54 69.96) (end 127.5 69.96) (width 0.254) (layer "F.Cu") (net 1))
 (segment (start 119.6 79.4) (end 123.2 75.8) (width 0.254) (layer "F.Cu") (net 1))
 (segment (start 123.2 75.8) (end 123.2 72.3) (width 0.254) (layer "F.Cu") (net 1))
 (segment (start 116.6 79.4) (end 119.6 79.4) (width 0.254) (layer "F.Cu") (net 1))
 (segment (start 133.5 70) (end 134 70) (width 0.254) (layer "F.Cu") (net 1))
 (segment (start 112 85.5) (end 112 84) (width 0.254) (layer "F.Cu") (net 1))
 (segment (start 127.54 70) (end 127.5 69.96) (width 0.254) (layer "F.Cu") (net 1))
 (segment (start 140 70.5) (end 144.5 70.5) (width 0.254) (layer "F.Cu") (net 1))
 (segment (start 123.2 72.3) (end 125.54 69.96) (width 0.254) (layer "F.Cu") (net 1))
 (segment (start 112 84) (end 116.6 79.4) (width 0.254) (layer "F.Cu") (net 1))
 (segment (start 133.5 70) (end 127.54 70) (width 0.254) (layer "F.Cu") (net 1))
 (segment (start 134 70) (end 134.5 70.5) (width 0.254) (layer "F.Cu") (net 1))
 (segment (start 147.42 54) (end 147.42 54.42) (width 0.254) (layer "F.Cu") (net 5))
 (segment (start 147.42 54.42) (end 153 60) (width 0.254) (layer "F.Cu") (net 5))
 (segment (start 153 60) (end 155.46 60) (width 0.254) (layer "F.Cu") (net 5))
 (segment (start 119.88 69.96) (end 119.88 72.5) (width 0.254) (layer "F.Cu") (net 10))
 (segment (start 112.015 59.015) (end 109 56) (width 0.254) (layer "F.Cu") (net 3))
 (segment (start 109 56) (end 108 56) (width 0.254) (layer "F.Cu") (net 3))
 (segment (start 115 59.015) (end 112.015 59.015) (width 0.254) (layer "F.Cu") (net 3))
 (segment (start 144.42 94.5) (end 146.44 96.52) (width 0.254) (layer "F.Cu") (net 8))
 (segment (start 162.620924 85.779076) (end 162.620924 78.220924) (width 0.254) (layer "F.Cu") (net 8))
 (segment (start 123.61 50.01) (end 123.61 48.77) (width 0.254) (layer "F.Cu") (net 8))
 (segment (start 146.44 96.52) (end 151.88 96.52) (width 0.254) (layer "F.Cu") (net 8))
 (segment (start 160 84.5) (end 160 85.2) (width 0.254) (layer "F.Cu") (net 8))
 (segment (start 160 85.2) (end 161.2 86.4) (width 0.254) (layer "F.Cu") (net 8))
 (segment (start 155.8 73.8) (end 133 51) (width 0.254) (layer "F.Cu") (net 8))
 (segment (start 134.6 50.2) (end 130.2 50.2) (width 0.254) (layer "F.Cu") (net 8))
 (segment (start 128.73 48.73) (end 128.6 48.86) (width 0.254) (layer "F.Cu") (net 8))
 (segment (start 162.6 85.8) (end 162.620924 85.779076) (width 0.254) (layer "F.Cu") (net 8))
 (segment (start 162 86.4) (end 162.6 85.8) (width 0.254) (layer "F.Cu") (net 8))
 (segment (start 162.620924 78.220924) (end 134.6 50.2) (width 0.254) (layer "F.Cu") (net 8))
 (segment (start 155.8 75.8) (end 155.8 73.8) (width 0.254) (layer "F.Cu") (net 8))
 (segment (start 130.2 50.2) (end 128.73 48.73) (width 0.254) (layer "F.Cu") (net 8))
 (segment (start 161.2 86.4) (end 162 86.4) (width 0.254) (layer "F.Cu") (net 8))
 (segment (start 160 80) (end 155.8 75.8) (width 0.254) (layer "F.Cu") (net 8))
 (segment (start 151.88 96.52) (end 162.6 85.8) (width 0.254) (layer "F.Cu") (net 8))
 (segment (start 124.6 51) (end 123.61 50.01) (width 0.254) (layer "F.Cu") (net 8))
 (segment (start 133 51) (end 124.6 51) (width 0.254) (layer "F.Cu") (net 8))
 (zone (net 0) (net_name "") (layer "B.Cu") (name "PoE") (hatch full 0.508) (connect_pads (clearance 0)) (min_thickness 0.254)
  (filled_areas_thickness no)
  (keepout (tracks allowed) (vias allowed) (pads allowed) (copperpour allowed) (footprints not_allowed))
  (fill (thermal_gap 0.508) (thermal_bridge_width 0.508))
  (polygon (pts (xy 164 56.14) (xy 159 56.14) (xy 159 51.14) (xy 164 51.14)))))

